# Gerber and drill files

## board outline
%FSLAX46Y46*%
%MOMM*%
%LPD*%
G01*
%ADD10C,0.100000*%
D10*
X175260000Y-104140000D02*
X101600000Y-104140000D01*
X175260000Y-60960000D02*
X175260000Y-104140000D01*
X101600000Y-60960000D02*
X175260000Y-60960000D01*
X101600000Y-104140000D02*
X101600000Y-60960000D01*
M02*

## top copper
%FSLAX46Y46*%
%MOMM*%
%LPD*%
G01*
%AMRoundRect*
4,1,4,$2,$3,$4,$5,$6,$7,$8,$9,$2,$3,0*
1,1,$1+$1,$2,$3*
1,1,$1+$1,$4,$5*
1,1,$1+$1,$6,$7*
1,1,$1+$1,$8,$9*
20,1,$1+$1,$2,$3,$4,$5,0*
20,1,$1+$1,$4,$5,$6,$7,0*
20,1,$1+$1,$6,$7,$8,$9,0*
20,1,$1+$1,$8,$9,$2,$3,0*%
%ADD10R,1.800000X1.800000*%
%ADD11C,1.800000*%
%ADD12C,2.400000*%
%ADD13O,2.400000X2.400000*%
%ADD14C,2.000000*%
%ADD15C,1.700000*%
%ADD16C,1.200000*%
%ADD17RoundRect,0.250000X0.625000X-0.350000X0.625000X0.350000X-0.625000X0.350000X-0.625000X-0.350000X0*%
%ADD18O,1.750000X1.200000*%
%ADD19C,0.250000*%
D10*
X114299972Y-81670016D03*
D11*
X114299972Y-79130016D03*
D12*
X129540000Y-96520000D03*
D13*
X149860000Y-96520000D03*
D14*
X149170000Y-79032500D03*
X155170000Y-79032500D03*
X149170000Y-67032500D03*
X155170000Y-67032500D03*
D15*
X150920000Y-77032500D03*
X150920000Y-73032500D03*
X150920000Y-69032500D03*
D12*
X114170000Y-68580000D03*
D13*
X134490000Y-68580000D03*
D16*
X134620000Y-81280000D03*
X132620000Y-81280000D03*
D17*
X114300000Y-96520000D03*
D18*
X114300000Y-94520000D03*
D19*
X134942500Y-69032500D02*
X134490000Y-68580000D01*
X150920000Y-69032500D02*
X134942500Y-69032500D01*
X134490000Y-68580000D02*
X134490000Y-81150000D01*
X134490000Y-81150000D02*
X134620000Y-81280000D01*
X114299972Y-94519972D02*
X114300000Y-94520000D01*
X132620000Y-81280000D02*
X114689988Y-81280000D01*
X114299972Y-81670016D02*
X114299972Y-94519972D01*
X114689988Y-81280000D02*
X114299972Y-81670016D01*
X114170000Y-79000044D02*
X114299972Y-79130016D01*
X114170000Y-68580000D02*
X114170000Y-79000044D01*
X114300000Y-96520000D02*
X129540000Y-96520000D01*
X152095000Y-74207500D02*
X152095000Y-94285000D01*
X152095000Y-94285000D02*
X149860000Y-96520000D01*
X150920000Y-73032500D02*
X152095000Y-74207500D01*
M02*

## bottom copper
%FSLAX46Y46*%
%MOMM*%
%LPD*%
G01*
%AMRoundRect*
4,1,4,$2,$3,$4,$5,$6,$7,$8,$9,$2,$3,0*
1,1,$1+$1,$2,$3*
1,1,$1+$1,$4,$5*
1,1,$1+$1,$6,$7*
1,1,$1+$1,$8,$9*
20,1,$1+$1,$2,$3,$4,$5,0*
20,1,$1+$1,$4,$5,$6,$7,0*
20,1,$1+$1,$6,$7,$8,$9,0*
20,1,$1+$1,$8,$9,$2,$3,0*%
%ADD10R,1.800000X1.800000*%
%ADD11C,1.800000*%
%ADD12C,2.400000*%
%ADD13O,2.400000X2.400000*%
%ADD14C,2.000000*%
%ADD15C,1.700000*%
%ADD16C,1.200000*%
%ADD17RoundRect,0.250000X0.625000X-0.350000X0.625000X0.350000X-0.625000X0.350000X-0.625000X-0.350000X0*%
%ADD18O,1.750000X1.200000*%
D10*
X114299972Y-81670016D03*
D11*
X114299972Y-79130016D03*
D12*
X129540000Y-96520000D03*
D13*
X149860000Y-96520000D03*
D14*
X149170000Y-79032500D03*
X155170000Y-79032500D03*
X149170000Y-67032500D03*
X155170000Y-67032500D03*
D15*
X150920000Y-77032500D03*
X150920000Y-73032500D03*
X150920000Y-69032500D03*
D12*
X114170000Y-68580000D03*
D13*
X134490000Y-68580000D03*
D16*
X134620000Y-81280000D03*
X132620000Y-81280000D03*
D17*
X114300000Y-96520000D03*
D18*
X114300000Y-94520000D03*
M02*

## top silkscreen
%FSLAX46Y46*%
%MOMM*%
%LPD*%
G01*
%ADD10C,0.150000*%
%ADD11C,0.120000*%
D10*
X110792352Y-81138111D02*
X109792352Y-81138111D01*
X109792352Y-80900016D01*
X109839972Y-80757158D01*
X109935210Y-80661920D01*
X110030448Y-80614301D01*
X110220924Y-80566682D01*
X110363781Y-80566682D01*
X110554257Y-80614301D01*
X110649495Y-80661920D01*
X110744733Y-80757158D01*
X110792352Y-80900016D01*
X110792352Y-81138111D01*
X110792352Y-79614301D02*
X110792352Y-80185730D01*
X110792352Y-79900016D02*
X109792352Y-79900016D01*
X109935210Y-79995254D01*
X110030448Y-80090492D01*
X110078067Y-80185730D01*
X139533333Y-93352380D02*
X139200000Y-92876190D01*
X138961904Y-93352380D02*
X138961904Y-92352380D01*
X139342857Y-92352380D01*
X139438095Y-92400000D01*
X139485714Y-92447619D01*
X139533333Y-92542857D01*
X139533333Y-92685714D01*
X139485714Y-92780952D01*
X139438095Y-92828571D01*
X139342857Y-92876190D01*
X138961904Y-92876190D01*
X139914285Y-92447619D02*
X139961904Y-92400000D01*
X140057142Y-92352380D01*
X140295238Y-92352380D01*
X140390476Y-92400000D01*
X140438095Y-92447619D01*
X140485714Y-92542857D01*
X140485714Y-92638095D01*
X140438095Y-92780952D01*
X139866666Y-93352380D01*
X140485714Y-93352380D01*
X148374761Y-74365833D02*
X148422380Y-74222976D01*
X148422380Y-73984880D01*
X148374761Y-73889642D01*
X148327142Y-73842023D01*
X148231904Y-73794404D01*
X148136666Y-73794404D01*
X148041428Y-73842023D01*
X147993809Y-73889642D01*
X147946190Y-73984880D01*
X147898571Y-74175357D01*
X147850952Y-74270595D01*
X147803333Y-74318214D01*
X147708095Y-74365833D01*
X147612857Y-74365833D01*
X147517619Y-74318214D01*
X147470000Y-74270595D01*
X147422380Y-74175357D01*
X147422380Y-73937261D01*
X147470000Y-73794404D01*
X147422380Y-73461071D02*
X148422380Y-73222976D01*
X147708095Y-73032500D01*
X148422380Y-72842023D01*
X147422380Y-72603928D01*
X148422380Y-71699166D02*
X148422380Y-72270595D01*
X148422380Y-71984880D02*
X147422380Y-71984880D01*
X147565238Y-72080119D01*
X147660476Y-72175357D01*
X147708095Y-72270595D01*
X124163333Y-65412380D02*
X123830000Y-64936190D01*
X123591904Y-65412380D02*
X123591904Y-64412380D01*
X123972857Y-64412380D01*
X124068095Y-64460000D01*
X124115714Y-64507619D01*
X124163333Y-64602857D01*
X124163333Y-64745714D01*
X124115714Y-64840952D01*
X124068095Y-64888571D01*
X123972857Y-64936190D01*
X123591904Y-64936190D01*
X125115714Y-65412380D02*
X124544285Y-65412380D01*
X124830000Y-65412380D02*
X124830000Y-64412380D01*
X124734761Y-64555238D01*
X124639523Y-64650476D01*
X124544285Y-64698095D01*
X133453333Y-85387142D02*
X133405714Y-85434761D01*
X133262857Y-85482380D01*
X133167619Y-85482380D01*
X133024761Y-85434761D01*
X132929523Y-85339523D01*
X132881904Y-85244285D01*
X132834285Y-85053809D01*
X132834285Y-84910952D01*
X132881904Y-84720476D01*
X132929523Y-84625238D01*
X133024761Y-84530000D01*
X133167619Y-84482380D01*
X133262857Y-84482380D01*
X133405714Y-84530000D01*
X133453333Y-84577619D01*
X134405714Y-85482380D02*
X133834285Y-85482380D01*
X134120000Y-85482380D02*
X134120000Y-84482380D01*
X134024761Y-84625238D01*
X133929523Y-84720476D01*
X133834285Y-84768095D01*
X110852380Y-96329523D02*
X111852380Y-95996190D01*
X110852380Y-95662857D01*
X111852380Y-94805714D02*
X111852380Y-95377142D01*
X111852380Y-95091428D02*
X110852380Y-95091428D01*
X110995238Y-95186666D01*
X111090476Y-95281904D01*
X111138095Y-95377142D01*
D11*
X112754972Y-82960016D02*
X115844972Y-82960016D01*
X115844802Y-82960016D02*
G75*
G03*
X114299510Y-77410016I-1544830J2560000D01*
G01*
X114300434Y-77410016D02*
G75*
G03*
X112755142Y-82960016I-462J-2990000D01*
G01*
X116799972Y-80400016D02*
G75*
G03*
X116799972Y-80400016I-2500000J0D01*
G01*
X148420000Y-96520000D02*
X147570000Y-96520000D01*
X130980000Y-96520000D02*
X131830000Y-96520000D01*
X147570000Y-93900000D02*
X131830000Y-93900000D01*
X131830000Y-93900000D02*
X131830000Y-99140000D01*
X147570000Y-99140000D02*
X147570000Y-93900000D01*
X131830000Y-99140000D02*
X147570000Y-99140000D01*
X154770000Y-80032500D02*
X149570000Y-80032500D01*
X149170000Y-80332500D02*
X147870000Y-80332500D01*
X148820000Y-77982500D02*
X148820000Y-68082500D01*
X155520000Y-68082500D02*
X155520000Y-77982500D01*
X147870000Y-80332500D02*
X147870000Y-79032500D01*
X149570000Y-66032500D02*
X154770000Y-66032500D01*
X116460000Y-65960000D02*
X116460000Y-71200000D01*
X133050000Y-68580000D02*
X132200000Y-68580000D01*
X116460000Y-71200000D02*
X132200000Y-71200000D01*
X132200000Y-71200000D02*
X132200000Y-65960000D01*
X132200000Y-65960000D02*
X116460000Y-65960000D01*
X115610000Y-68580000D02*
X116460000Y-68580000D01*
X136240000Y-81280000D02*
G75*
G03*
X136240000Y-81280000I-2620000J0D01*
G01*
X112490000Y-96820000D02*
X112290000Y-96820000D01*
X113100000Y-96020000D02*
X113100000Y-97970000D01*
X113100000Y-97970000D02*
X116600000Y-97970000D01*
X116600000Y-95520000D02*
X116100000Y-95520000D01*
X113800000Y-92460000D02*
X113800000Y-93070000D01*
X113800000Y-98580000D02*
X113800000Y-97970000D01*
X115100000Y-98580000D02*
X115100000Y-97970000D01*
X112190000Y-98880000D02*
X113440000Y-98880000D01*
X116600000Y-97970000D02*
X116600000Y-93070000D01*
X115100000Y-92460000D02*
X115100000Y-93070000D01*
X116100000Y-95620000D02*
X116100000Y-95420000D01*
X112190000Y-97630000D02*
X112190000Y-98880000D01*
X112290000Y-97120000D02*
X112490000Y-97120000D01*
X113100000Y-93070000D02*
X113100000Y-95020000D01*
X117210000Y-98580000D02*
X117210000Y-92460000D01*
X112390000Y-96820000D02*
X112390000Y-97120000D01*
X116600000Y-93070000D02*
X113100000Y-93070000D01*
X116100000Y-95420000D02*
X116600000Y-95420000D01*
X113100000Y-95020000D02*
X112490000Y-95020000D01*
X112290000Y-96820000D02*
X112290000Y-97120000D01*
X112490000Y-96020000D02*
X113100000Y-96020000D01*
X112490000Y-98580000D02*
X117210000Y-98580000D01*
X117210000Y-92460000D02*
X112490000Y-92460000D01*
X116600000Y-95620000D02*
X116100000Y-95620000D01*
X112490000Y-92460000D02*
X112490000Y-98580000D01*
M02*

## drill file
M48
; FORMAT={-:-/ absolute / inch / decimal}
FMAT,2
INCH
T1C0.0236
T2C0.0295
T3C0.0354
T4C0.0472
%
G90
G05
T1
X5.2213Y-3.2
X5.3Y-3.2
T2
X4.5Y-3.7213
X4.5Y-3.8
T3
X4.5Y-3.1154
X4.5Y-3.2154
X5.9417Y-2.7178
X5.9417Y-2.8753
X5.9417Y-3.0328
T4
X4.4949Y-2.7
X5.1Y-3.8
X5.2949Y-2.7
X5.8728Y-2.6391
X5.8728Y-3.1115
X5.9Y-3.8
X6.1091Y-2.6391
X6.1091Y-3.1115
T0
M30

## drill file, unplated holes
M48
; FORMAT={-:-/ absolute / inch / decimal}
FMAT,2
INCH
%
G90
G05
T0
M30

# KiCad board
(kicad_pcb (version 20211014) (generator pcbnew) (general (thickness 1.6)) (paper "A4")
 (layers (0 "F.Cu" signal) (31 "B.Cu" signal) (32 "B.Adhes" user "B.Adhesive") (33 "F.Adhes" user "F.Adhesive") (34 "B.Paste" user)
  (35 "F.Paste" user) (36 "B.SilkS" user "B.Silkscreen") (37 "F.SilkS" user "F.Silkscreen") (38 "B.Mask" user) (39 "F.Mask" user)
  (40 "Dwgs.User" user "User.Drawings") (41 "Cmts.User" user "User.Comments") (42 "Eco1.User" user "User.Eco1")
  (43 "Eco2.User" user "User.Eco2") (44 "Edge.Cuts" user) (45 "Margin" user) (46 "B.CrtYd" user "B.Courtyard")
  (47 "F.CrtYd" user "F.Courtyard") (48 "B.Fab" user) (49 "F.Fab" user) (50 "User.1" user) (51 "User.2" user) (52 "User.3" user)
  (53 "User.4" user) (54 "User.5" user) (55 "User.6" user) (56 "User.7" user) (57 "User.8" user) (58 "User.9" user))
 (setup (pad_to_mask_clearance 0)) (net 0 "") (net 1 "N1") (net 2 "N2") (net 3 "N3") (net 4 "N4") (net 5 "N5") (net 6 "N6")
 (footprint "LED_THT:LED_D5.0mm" (layer "F.Cu") (at 114.299972 81.670016 90)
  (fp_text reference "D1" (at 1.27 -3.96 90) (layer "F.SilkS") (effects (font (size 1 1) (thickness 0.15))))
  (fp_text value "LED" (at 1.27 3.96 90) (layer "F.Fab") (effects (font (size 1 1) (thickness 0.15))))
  (fp_line (start -1.29 -1.545) (end -1.29 1.545) (layer "F.SilkS") (width 0.12))
  (fp_arc (start 4.26 -0.000462) (mid 2.072002 2.880433) (end -1.29 1.54483) (layer "F.SilkS") (width 0.12))
  (fp_arc (start -1.29 -1.54483) (mid 2.072002 -2.880433) (end 4.26 0.000462) (layer "F.SilkS") (width 0.12))
  (fp_circle (center 1.27 0) (end 3.77 0) (layer "F.SilkS") (width 0.12) (fill none))
  (pad "1" thru_hole rect (at 0 0 90) (size 1.8 1.8) (drill 0.9) (layers *.Cu *.Mask) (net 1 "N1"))
  (pad "2" thru_hole circle (at 2.54 0 90) (size 1.8 1.8) (drill 0.9) (layers *.Cu *.Mask) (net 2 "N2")))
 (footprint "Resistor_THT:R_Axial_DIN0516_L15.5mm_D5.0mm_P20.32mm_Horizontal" (layer "F.Cu") (at 129.54 96.52)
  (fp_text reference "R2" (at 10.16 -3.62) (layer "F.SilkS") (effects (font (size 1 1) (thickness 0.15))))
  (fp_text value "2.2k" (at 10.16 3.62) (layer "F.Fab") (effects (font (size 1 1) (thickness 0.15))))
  (fp_line (start 18.88 0) (end 18.03 0) (layer "F.SilkS") (width 0.12))
  (fp_line (start 1.44 0) (end 2.29 0) (layer "F.SilkS") (width 0.12))
  (fp_line (start 18.03 -2.62) (end 2.29 -2.62) (layer "F.SilkS") (width 0.12))
  (fp_line (start 2.29 -2.62) (end 2.29 2.62) (layer "F.SilkS") (width 0.12))
  (fp_line (start 18.03 2.62) (end 18.03 -2.62) (layer "F.SilkS") (width 0.12))
  (fp_line (start 2.29 2.62) (end 18.03 2.62) (layer "F.SilkS") (width 0.12))
  (pad "1" thru_hole circle (at 0 0) (size 2.4 2.4) (drill 1.2) (layers *.Cu *.Mask) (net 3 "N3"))
  (pad "2" thru_hole oval (at 20.32 0) (size 2.4 2.4) (drill 1.2) (layers *.Cu *.Mask) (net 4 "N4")))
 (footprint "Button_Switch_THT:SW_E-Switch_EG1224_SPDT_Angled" (layer "F.Cu") (at 150.92 77.0325 90)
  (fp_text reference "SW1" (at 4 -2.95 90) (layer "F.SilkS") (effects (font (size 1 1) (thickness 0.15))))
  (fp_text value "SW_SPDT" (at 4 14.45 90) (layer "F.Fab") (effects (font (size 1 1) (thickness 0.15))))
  (fp_line (start -3 3.85) (end -3 -1.35) (layer "F.SilkS") (width 0.12))
  (fp_line (start -3.3 -1.75) (end -3.3 -3.05) (layer "F.SilkS") (width 0.12))
  (fp_line (start -0.95 -2.1) (end 8.95 -2.1) (layer "F.SilkS") (width 0.12))
  (fp_line (start 8.95 4.6) (end -0.95 4.6) (layer "F.SilkS") (width 0.12))
  (fp_line (start -3.3 -3.05) (end -2 -3.05) (layer "F.SilkS") (width 0.12))
  (fp_line (start 11 -1.35) (end 11 3.85) (layer "F.SilkS") (width 0.12))
  (pad "" thru_hole circle (at -2 -1.75 90) (size 2 2) (drill 1.2) (layers *.Cu *.Mask))
  (pad "" thru_hole circle (at -2 4.25 90) (size 2 2) (drill 1.2) (layers *.Cu *.Mask))
  (pad "" thru_hole circle (at 10 -1.75 90) (size 2 2) (drill 1.2) (layers *.Cu *.Mask))
  (pad "" thru_hole circle (at 10 4.25 90) (size 2 2) (drill 1.2) (layers *.Cu *.Mask))
  (pad "1" thru_hole circle (at 0 0 90) (size 1.7 1.7) (drill 0.9) (layers *.Cu *.Mask) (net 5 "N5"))
  (pad "2" thru_hole circle (at 4 0 90) (size 1.7 1.7) (drill 0.9) (layers *.Cu *.Mask) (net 4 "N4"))
  (pad "3" thru_hole circle (at 8 0 90) (size 1.7 1.7) (drill 0.9) (layers *.Cu *.Mask) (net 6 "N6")))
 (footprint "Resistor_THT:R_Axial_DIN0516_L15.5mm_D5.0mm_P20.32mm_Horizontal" (layer "F.Cu") (at 114.17 68.58)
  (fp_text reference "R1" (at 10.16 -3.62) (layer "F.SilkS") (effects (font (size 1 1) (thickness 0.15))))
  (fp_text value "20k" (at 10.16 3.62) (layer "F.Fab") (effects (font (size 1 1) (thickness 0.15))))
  (fp_line (start 2.29 -2.62) (end 2.29 2.62) (layer "F.SilkS") (width 0.12))
  (fp_line (start 18.88 0) (end 18.03 0) (layer "F.SilkS") (width 0.12))
  (fp_line (start 2.29 2.62) (end 18.03 2.62) (layer "F.SilkS") (width 0.12))
  (fp_line (start 18.03 2.62) (end 18.03 -2.62) (layer "F.SilkS") (width 0.12))
  (fp_line (start 18.03 -2.62) (end 2.29 -2.62) (layer "F.SilkS") (width 0.12))
  (fp_line (start 1.44 0) (end 2.29 0) (layer "F.SilkS") (width 0.12))
  (pad "1" thru_hole circle (at 0 0) (size 2.4 2.4) (drill 1.2) (layers *.Cu *.Mask) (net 2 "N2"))
  (pad "2" thru_hole oval (at 20.32 0) (size 2.4 2.4) (drill 1.2) (layers *.Cu *.Mask) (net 6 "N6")))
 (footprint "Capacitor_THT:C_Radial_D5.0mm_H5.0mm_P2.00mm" (layer "F.Cu") (at 134.62 81.28 180)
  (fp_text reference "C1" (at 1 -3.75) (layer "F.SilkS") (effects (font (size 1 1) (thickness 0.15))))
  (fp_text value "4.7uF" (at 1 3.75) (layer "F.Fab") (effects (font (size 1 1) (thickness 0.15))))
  (fp_circle (center 1 0) (end 3.62 0) (layer "F.SilkS") (width 0.12) (fill none))
  (pad "1" thru_hole circle (at 0 0 180) (size 1.2 1.2) (drill 0.6) (layers *.Cu *.Mask) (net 6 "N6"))
  (pad "2" thru_hole circle (at 2 0 180) (size 1.2 1.2) (drill 0.6) (layers *.Cu *.Mask) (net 1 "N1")))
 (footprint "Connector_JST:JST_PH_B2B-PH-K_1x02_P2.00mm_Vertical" (layer "F.Cu") (at 114.3 96.52 90)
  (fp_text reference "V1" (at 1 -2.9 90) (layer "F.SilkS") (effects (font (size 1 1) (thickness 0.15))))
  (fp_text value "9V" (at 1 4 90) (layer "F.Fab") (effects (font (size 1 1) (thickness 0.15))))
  (fp_line (start -0.3 -1.81) (end -0.3 -2.01) (layer "F.SilkS") (width 0.12))
  (fp_line (start 0.5 -1.2) (end -1.45 -1.2) (layer "F.SilkS") (width 0.12))
  (fp_line (start -1.45 -1.2) (end -1.45 2.3) (layer "F.SilkS") (width 0.12))
  (fp_line (start 1 2.3) (end 1 1.8) (layer "F.SilkS") (width 0.12))
  (fp_line (start 4.06 -0.5) (end 3.45 -0.5) (layer "F.SilkS") (width 0.12))
  (fp_line (start -2.06 -0.5) (end -1.45 -0.5) (layer "F.SilkS") (width 0.12))
  (fp_line (start -2.06 0.8) (end -1.45 0.8) (layer "F.SilkS") (width 0.12))
  (fp_line (start -2.36 -2.11) (end -2.36 -0.86) (layer "F.SilkS") (width 0.12))
  (fp_line (start -1.45 2.3) (end 3.45 2.3) (layer "F.SilkS") (width 0.12))
  (fp_line (start 4.06 0.8) (end 3.45 0.8) (layer "F.SilkS") (width 0.12))
  (fp_line (start 0.9 1.8) (end 1.1 1.8) (layer "F.SilkS") (width 0.12))
  (fp_line (start -1.11 -2.11) (end -2.36 -2.11) (layer "F.SilkS") (width 0.12))
  (fp_line (start -0.6 -2.01) (end -0.6 -1.81) (layer "F.SilkS") (width 0.12))
  (fp_line (start 3.45 -1.2) (end 1.5 -1.2) (layer "F.SilkS") (width 0.12))
  (fp_line (start -2.06 2.91) (end 4.06 2.91) (layer "F.SilkS") (width 0.12))
  (fp_line (start -0.3 -1.91) (end -0.6 -1.91) (layer "F.SilkS") (width 0.12))
  (fp_line (start 3.45 2.3) (end 3.45 -1.2) (layer "F.SilkS") (width 0.12))
  (fp_line (start 1.1 1.8) (end 1.1 2.3) (layer "F.SilkS") (width 0.12))
  (fp_line (start 1.5 -1.2) (end 1.5 -1.81) (layer "F.SilkS") (width 0.12))
  (fp_line (start -0.3 -2.01) (end -0.6 -2.01) (layer "F.SilkS") (width 0.12))
  (fp_line (start 0.5 -1.81) (end 0.5 -1.2) (layer "F.SilkS") (width 0.12))
  (fp_line (start -2.06 -1.81) (end -2.06 2.91) (layer "F.SilkS") (width 0.12))
  (fp_line (start 4.06 2.91) (end 4.06 -1.81) (layer "F.SilkS") (width 0.12))
  (fp_line (start 0.9 2.3) (end 0.9 1.8) (layer "F.SilkS") (width 0.12))
  (fp_line (start 4.06 -1.81) (end -2.06 -1.81) (layer "F.SilkS") (width 0.12))
  (pad "1" thru_hole roundrect (at 0 0 90) (size 1.2 1.75) (drill 0.75) (layers *.Cu *.Mask) (roundrect_rratio 0.2083333333) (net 3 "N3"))
  (pad "2" thru_hole oval (at 2 0 90) (size 1.2 1.75) (drill 0.75) (layers *.Cu *.Mask) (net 1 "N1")))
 (gr_line (start 175.26 104.14) (end 101.6 104.14) (layer "Edge.Cuts") (width 0.1))
 (gr_line (start 175.26 60.96) (end 175.26 104.14) (layer "Edge.Cuts") (width 0.1))
 (gr_line (start 101.6 60.96) (end 175.26 60.96) (layer "Edge.Cuts") (width 0.1))
 (gr_line (start 101.6 104.14) (end 101.6 60.96) (layer "Edge.Cuts") (width 0.1))
 (segment (start 134.9425 69.0325) (end 134.49 68.58) (width 0.25) (layer "F.Cu") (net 6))
 (segment (start 150.92 69.0325) (end 134.9425 69.0325) (width 0.25) (layer "F.Cu") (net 6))
 (segment (start 134.49 68.58) (end 134.49 81.15) (width 0.25) (layer "F.Cu") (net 6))
 (segment (start 134.49 81.15) (end 134.62 81.28) (width 0.25) (layer "F.Cu") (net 6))
 (segment (start 114.299972 94.519972) (end 114.3 94.52) (width 0.25) (layer "F.Cu") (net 1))
 (segment (start 132.62 81.28) (end 114.689988 81.28) (width 0.25) (layer "F.Cu") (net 1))
 (segment (start 114.299972 81.670016) (end 114.299972 94.519972) (width 0.25) (layer "F.Cu") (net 1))
 (segment (start 114.689988 81.28) (end 114.299972 81.670016) (width 0.25) (layer "F.Cu") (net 1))
 (segment (start 114.17 79.000044) (end 114.299972 79.130016) (width 0.25) (layer "F.Cu") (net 2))
 (segment (start 114.17 68.58) (end 114.17 79.000044) (width 0.25) (layer "F.Cu") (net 2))
 (segment (start 114.3 96.52) (end 129.54 96.52) (width 0.25) (layer "F.Cu") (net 3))
 (segment (start 152.095 74.2075) (end 152.095 94.285) (width 0.25) (layer "F.Cu") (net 4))
 (segment (start 152.095 94.285) (end 149.86 96.52) (width 0.25) (layer "F.Cu") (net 4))
 (segment (start 150.92 73.0325) (end 152.095 74.2075) (width 0.25) (layer "F.Cu") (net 4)))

